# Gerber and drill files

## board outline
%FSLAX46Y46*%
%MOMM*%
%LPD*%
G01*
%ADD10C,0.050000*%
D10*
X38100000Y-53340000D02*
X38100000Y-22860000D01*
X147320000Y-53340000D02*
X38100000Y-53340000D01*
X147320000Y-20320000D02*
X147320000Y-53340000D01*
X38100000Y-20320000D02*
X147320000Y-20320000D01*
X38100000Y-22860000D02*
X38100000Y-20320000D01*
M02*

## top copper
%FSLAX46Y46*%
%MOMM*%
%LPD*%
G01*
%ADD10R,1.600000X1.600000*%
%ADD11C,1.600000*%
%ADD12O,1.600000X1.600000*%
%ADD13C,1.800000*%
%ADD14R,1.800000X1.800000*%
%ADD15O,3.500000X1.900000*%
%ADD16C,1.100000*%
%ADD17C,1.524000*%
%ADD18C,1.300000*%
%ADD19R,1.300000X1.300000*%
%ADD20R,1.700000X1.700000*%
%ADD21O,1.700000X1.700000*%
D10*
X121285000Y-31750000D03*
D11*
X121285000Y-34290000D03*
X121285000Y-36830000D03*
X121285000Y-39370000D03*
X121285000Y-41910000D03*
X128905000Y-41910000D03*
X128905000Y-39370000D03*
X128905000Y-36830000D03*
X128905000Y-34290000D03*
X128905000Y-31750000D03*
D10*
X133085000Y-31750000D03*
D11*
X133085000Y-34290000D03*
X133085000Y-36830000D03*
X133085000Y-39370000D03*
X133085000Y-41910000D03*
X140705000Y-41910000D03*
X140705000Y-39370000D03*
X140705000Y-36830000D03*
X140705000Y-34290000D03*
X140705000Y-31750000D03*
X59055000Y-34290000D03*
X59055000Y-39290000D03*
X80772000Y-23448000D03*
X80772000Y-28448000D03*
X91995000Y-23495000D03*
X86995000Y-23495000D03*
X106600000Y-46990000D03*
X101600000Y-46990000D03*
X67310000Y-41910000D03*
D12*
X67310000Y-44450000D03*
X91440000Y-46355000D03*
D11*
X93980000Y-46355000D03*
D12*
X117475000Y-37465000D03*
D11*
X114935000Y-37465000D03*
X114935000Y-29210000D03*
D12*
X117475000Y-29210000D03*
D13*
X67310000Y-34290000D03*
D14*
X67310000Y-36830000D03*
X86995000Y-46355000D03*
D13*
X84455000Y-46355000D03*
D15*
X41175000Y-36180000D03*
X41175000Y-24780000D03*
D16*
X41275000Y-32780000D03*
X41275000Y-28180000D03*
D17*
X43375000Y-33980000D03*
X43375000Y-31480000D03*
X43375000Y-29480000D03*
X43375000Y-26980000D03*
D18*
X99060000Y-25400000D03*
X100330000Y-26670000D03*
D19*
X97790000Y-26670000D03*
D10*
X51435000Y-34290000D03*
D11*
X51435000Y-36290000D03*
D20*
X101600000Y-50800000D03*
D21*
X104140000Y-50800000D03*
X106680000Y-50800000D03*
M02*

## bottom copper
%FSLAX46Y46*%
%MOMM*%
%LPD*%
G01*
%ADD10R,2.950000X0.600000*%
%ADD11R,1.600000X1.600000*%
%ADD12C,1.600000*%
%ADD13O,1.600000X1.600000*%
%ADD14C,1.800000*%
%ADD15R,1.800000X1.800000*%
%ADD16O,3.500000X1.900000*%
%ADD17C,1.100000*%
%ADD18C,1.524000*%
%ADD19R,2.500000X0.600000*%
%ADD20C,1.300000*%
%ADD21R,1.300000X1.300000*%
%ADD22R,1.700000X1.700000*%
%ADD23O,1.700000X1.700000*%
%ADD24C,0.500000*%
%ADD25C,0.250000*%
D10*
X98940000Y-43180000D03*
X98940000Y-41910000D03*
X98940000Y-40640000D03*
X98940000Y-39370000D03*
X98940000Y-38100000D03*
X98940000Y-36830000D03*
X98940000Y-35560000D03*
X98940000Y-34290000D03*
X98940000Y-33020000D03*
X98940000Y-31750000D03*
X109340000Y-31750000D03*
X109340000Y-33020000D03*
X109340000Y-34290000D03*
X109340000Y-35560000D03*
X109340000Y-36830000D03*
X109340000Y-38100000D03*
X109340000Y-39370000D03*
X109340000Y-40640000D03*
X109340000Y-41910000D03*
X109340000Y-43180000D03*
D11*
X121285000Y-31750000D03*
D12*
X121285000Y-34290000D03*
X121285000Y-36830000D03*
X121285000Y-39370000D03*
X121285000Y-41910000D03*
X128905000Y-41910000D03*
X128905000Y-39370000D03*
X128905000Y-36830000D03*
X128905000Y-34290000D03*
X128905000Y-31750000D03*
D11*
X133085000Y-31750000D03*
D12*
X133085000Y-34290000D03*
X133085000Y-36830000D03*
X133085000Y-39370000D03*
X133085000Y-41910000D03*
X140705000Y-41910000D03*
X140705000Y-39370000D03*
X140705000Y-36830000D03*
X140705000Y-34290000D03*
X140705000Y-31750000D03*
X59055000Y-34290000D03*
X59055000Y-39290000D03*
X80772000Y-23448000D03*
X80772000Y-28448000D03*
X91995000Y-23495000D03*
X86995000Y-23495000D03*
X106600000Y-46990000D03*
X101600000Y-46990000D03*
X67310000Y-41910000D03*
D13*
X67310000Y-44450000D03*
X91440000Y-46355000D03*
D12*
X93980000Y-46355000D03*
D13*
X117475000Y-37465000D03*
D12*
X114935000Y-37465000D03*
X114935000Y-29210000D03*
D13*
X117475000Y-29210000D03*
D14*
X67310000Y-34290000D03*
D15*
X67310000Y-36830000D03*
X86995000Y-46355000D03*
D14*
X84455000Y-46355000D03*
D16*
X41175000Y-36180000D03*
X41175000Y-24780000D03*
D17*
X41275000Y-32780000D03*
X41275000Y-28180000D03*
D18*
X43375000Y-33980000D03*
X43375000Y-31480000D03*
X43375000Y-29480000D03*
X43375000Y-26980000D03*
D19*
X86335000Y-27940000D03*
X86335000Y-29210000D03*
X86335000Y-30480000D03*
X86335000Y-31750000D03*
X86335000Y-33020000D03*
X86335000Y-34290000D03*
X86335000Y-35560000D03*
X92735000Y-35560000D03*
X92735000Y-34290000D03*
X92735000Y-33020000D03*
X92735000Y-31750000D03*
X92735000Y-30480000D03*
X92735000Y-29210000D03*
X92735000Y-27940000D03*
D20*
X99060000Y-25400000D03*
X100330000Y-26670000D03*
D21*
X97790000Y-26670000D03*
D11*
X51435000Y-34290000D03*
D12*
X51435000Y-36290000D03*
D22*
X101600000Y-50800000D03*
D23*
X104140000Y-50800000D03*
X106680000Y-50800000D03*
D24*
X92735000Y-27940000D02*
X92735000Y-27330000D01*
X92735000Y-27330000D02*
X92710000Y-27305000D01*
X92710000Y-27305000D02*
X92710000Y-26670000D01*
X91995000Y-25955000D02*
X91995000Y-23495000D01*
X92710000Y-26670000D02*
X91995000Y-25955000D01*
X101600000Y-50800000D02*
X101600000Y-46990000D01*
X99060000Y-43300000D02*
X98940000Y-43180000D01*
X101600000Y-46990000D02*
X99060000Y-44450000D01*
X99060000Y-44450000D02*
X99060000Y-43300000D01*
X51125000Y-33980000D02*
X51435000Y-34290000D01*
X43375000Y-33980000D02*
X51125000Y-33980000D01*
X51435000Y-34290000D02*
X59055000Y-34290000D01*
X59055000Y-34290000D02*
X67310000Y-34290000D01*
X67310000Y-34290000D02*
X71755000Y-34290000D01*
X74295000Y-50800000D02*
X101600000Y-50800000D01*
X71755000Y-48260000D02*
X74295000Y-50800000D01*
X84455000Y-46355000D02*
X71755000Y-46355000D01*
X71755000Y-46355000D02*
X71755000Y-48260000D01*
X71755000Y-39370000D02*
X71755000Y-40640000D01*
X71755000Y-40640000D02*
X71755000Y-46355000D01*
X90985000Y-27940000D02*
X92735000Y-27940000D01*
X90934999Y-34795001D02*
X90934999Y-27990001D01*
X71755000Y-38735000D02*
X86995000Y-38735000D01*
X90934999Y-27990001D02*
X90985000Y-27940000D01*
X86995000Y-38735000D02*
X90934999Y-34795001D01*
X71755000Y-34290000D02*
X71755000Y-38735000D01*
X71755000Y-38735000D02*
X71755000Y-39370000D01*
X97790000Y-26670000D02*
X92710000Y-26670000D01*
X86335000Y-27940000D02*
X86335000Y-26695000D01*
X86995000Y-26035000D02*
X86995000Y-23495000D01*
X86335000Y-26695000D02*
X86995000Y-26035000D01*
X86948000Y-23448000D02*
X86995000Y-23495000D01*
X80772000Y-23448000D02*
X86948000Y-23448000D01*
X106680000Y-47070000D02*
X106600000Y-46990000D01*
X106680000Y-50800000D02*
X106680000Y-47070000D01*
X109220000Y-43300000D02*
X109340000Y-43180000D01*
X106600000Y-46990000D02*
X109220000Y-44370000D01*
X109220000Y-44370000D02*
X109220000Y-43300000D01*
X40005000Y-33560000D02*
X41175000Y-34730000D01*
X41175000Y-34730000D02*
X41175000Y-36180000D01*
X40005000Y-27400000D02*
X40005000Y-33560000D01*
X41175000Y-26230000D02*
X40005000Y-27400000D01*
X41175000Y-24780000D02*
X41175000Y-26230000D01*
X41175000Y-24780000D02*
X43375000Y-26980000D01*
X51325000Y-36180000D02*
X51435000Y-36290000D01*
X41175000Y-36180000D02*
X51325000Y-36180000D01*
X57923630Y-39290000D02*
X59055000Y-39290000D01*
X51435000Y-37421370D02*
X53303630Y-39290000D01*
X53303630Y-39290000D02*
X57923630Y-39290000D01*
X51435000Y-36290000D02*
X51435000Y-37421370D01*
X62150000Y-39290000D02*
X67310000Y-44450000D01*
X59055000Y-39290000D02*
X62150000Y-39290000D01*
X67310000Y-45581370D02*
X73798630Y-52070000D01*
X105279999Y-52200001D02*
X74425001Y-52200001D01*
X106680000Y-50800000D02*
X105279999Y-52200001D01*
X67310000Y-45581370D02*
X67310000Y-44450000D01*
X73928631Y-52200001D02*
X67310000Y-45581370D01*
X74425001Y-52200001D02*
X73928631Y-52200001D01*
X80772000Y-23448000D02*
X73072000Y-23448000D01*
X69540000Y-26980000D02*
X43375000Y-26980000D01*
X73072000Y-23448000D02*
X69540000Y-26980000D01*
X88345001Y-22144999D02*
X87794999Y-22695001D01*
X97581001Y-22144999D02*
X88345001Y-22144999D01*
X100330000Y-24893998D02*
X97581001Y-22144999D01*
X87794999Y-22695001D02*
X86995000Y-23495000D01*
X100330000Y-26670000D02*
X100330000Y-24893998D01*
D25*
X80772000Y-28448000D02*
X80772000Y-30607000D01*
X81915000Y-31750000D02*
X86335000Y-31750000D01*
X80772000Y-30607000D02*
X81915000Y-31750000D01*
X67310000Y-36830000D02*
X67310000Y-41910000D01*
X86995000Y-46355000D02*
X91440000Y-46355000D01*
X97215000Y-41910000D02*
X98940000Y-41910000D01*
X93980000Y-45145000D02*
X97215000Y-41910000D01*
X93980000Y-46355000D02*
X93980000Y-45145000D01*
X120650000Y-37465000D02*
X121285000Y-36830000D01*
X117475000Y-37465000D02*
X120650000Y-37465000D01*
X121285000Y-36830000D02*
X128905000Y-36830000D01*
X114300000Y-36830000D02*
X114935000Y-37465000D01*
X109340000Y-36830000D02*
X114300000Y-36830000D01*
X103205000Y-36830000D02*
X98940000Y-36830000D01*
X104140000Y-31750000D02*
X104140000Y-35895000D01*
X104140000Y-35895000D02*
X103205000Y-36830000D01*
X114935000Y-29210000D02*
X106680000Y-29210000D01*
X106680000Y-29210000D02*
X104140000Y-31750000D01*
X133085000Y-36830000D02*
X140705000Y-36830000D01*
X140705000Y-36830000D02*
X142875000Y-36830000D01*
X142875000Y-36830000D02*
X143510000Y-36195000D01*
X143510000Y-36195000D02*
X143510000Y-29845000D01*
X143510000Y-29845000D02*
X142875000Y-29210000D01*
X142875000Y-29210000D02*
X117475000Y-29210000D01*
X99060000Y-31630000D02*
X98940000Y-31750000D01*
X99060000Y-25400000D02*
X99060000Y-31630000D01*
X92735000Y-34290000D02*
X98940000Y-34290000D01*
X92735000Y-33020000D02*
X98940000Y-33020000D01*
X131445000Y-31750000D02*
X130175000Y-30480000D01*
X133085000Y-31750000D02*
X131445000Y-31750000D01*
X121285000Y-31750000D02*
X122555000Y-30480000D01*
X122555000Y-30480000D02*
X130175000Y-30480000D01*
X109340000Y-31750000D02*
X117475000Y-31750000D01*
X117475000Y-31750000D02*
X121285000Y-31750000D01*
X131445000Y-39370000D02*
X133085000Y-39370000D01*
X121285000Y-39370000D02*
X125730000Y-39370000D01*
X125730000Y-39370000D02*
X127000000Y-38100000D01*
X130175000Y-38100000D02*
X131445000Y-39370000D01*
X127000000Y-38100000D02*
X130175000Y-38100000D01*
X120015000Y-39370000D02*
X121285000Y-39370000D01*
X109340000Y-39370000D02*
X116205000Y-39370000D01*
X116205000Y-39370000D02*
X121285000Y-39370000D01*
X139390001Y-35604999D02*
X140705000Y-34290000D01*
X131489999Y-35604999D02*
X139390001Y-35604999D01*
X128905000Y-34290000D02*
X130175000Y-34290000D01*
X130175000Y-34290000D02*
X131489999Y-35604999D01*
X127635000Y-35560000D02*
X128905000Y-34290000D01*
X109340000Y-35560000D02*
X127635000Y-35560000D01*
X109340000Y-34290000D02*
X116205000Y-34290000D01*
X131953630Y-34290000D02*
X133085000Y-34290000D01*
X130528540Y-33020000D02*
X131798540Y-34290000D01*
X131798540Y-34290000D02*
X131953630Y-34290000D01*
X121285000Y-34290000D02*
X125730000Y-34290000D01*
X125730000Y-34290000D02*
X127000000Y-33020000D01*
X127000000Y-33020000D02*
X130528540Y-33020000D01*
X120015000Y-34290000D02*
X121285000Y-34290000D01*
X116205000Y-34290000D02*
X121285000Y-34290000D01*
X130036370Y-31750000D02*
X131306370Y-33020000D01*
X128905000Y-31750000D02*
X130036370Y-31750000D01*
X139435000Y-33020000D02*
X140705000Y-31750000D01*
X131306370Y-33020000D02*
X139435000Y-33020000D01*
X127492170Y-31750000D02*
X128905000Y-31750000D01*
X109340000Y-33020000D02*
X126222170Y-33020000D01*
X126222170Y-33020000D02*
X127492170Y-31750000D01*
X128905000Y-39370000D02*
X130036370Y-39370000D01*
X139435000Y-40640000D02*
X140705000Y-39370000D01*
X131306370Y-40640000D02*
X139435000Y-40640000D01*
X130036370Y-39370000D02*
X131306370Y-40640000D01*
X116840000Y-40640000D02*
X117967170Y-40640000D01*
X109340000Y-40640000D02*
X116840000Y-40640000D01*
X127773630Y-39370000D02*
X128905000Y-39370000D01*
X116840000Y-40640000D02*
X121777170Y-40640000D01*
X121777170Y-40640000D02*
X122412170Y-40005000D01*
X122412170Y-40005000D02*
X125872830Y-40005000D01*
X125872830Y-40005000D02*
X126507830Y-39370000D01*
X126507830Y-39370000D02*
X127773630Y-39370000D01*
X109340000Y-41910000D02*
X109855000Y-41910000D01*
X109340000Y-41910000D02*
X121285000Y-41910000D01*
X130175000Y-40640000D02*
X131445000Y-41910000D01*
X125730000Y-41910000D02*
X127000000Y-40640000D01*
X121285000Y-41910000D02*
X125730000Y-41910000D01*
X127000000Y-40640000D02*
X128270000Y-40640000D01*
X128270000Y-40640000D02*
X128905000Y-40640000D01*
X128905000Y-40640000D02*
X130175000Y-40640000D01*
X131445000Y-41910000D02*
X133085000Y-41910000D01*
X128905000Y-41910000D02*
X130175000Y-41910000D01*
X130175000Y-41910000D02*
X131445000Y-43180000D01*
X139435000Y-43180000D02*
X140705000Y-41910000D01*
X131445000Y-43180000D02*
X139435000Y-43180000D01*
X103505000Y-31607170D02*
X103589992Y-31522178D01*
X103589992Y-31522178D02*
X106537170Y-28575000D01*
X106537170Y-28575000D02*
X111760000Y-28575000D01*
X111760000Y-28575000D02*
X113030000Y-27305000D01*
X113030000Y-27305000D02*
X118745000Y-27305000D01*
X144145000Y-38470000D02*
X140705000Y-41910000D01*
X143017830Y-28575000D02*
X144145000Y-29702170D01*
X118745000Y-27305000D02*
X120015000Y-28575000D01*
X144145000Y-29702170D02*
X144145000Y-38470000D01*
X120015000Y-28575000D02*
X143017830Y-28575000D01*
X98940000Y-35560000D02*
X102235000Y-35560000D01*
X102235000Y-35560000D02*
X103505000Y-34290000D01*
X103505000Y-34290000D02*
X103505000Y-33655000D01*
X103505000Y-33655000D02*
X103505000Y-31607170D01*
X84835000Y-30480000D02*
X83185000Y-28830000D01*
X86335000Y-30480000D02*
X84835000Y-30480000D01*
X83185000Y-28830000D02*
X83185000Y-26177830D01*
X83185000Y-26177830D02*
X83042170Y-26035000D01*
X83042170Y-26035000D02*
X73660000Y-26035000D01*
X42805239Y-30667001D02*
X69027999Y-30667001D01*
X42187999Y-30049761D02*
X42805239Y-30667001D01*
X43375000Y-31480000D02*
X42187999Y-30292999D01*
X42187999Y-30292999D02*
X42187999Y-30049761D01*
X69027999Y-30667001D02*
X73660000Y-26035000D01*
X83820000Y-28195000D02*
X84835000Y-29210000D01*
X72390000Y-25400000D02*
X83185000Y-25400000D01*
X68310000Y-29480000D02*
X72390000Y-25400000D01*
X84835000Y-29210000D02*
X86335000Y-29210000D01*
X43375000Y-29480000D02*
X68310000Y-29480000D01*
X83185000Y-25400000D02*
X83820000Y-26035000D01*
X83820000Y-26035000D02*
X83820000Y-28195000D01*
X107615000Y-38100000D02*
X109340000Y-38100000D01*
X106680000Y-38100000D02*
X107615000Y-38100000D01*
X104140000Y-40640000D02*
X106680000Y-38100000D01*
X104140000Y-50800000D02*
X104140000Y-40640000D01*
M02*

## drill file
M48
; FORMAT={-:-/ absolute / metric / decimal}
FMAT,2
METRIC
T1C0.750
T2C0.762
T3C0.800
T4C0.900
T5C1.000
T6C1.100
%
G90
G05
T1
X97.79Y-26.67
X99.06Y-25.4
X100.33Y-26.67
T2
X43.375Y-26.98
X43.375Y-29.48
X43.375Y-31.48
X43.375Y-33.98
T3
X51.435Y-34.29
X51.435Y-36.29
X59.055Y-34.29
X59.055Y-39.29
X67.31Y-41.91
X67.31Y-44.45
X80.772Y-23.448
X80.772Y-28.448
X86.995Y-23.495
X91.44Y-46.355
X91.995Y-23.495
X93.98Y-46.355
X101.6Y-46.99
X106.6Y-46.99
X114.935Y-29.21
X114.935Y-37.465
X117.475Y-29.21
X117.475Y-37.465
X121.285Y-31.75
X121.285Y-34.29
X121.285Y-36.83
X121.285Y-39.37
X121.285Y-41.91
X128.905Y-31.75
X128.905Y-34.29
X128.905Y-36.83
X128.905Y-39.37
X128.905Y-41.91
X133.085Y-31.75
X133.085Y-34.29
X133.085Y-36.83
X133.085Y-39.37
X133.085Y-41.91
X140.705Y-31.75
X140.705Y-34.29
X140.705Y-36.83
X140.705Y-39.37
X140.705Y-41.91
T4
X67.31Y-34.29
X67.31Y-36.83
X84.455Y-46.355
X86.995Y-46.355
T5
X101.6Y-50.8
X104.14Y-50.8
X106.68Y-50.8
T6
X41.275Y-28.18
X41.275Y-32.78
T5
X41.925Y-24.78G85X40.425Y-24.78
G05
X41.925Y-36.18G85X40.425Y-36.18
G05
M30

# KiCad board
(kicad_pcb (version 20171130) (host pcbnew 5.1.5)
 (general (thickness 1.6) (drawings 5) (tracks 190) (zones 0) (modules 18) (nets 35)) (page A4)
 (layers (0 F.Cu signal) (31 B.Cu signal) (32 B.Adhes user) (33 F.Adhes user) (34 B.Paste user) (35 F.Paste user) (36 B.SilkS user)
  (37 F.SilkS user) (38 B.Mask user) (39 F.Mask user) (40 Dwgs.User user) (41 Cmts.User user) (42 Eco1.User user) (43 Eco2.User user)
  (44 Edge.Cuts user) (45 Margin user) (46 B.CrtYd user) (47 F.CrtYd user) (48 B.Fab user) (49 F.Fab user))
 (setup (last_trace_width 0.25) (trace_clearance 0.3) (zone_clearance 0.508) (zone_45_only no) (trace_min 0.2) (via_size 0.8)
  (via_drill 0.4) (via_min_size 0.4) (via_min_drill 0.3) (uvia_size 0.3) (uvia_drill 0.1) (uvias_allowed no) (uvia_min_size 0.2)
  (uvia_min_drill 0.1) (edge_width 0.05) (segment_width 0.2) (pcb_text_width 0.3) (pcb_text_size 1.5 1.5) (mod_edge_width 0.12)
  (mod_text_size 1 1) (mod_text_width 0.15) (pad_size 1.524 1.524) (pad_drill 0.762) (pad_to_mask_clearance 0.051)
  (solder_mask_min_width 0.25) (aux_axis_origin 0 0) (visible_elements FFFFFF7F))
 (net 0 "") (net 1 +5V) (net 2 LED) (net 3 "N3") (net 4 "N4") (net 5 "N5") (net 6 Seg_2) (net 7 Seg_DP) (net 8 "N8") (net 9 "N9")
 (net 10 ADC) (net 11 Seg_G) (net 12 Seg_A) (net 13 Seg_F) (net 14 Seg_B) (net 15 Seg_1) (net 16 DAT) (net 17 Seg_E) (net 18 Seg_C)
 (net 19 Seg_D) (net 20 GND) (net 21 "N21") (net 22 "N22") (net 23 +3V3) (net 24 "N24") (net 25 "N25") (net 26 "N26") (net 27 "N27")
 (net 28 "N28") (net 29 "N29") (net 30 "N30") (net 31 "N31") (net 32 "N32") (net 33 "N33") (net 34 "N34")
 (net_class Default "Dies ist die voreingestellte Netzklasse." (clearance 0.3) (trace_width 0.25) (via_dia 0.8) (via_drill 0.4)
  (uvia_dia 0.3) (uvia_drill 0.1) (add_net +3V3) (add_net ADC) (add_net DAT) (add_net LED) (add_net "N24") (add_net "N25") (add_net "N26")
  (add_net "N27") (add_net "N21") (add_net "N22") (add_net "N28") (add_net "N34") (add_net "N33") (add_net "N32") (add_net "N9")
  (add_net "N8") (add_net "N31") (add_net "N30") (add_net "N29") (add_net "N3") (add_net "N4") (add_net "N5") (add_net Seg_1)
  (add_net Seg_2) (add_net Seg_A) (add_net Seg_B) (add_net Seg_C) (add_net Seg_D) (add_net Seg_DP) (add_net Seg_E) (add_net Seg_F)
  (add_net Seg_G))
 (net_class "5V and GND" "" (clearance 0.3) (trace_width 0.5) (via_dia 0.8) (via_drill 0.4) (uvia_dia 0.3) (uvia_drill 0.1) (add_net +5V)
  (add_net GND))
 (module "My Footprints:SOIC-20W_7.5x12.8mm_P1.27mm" (layer B.Cu) (at 104.14 37.465)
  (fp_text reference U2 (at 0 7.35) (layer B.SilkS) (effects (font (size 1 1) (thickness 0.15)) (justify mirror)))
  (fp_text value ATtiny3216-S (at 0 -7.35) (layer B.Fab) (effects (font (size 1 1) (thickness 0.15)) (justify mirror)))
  (pad 1 smd rect (at -5.2 5.715) (size 2.95 0.6) (layers B.Cu B.Paste B.Mask) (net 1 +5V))
  (pad 2 smd rect (at -5.2 4.445) (size 2.95 0.6) (layers B.Cu B.Paste B.Mask) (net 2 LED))
  (pad 3 smd rect (at -5.2 3.175) (size 2.95 0.6) (layers B.Cu B.Paste B.Mask) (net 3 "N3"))
  (pad 4 smd rect (at -5.2 1.905) (size 2.95 0.6) (layers B.Cu B.Paste B.Mask) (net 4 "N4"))
  (pad 5 smd rect (at -5.2 0.635) (size 2.95 0.6) (layers B.Cu B.Paste B.Mask) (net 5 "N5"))
  (pad 6 smd rect (at -5.2 -0.635) (size 2.95 0.6) (layers B.Cu B.Paste B.Mask) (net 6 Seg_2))
  (pad 7 smd rect (at -5.2 -1.905) (size 2.95 0.6) (layers B.Cu B.Paste B.Mask) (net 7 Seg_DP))
  (pad 8 smd rect (at -5.2 -3.175) (size 2.95 0.6) (layers B.Cu B.Paste B.Mask) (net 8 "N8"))
  (pad 9 smd rect (at -5.2 -4.445) (size 2.95 0.6) (layers B.Cu B.Paste B.Mask) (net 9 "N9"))
  (pad 10 smd rect (at -5.2 -5.715) (size 2.95 0.6) (layers B.Cu B.Paste B.Mask) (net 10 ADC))
  (pad 11 smd rect (at 5.2 -5.715) (size 2.95 0.6) (layers B.Cu B.Paste B.Mask) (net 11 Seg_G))
  (pad 12 smd rect (at 5.2 -4.445) (size 2.95 0.6) (layers B.Cu B.Paste B.Mask) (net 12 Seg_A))
  (pad 13 smd rect (at 5.2 -3.175) (size 2.95 0.6) (layers B.Cu B.Paste B.Mask) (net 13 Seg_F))
  (pad 14 smd rect (at 5.2 -1.905) (size 2.95 0.6) (layers B.Cu B.Paste B.Mask) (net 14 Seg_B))
  (pad 15 smd rect (at 5.2 -0.635) (size 2.95 0.6) (layers B.Cu B.Paste B.Mask) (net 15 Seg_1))
  (pad 16 smd rect (at 5.2 0.635) (size 2.95 0.6) (layers B.Cu B.Paste B.Mask) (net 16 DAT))
  (pad 17 smd rect (at 5.2 1.905) (size 2.95 0.6) (layers B.Cu B.Paste B.Mask) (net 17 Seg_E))
  (pad 18 smd rect (at 5.2 3.175) (size 2.95 0.6) (layers B.Cu B.Paste B.Mask) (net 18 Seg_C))
  (pad 19 smd rect (at 5.2 4.445) (size 2.95 0.6) (layers B.Cu B.Paste B.Mask) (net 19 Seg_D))
  (pad 20 smd rect (at 5.2 5.715) (size 2.95 0.6) (layers B.Cu B.Paste B.Mask) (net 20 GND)))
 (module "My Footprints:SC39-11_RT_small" (layer F.Cu) (at 121.285 31.75)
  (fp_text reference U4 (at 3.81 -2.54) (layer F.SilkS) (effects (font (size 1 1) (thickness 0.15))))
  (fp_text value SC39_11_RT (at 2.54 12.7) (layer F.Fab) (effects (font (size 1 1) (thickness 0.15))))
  (pad 1 thru_hole rect (at 0 0) (size 1.6 1.6) (drill 0.8) (layers *.Cu *.Mask) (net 11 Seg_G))
  (pad 2 thru_hole circle (at 0 2.54) (size 1.6 1.6) (drill 0.8) (layers *.Cu *.Mask) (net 13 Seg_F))
  (pad 3 thru_hole circle (at 0 5.08) (size 1.6 1.6) (drill 0.8) (layers *.Cu *.Mask) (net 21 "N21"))
  (pad 4 thru_hole circle (at 0 7.62) (size 1.6 1.6) (drill 0.8) (layers *.Cu *.Mask) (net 17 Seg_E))
  (pad 5 thru_hole circle (at 0 10.16) (size 1.6 1.6) (drill 0.8) (layers *.Cu *.Mask) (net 19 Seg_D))
  (pad 6 thru_hole circle (at 7.62 10.16) (size 1.6 1.6) (drill 0.8) (layers *.Cu *.Mask) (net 7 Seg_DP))
  (pad 7 thru_hole circle (at 7.62 7.62) (size 1.6 1.6) (drill 0.8) (layers *.Cu *.Mask) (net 18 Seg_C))
  (pad 8 thru_hole circle (at 7.62 5.08) (size 1.6 1.6) (drill 0.8) (layers *.Cu *.Mask) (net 21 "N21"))
  (pad 9 thru_hole circle (at 7.62 2.54) (size 1.6 1.6) (drill 0.8) (layers *.Cu *.Mask) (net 14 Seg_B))
  (pad 10 thru_hole circle (at 7.62 0) (size 1.6 1.6) (drill 0.8) (layers *.Cu *.Mask) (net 12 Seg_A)))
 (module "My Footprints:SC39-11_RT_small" (layer F.Cu) (at 133.085 31.75)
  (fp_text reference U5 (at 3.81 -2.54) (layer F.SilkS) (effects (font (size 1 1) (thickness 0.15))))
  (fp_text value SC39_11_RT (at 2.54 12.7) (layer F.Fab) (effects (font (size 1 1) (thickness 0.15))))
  (pad 1 thru_hole rect (at 0 0) (size 1.6 1.6) (drill 0.8) (layers *.Cu *.Mask) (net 11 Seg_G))
  (pad 2 thru_hole circle (at 0 2.54) (size 1.6 1.6) (drill 0.8) (layers *.Cu *.Mask) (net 13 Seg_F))
  (pad 3 thru_hole circle (at 0 5.08) (size 1.6 1.6) (drill 0.8) (layers *.Cu *.Mask) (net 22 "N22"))
  (pad 4 thru_hole circle (at 0 7.62) (size 1.6 1.6) (drill 0.8) (layers *.Cu *.Mask) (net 17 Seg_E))
  (pad 5 thru_hole circle (at 0 10.16) (size 1.6 1.6) (drill 0.8) (layers *.Cu *.Mask) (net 19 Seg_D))
  (pad 6 thru_hole circle (at 7.62 10.16) (size 1.6 1.6) (drill 0.8) (layers *.Cu *.Mask) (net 7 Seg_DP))
  (pad 7 thru_hole circle (at 7.62 7.62) (size 1.6 1.6) (drill 0.8) (layers *.Cu *.Mask) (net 18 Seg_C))
  (pad 8 thru_hole circle (at 7.62 5.08) (size 1.6 1.6) (drill 0.8) (layers *.Cu *.Mask) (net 22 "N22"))
  (pad 9 thru_hole circle (at 7.62 2.54) (size 1.6 1.6) (drill 0.8) (layers *.Cu *.Mask) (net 14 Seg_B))
  (pad 10 thru_hole circle (at 7.62 0) (size 1.6 1.6) (drill 0.8) (layers *.Cu *.Mask) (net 12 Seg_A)))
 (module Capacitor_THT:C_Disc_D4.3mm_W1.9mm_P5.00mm (layer F.Cu) (at 59.055 34.29 270)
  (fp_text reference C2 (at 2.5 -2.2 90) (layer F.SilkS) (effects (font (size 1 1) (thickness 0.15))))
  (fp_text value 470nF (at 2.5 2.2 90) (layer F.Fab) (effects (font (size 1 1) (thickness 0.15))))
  (pad 1 thru_hole circle (at 0 0 270) (size 1.6 1.6) (drill 0.8) (layers *.Cu *.Mask) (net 1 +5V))
  (pad 2 thru_hole circle (at 5 0 270) (size 1.6 1.6) (drill 0.8) (layers *.Cu *.Mask) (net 20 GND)))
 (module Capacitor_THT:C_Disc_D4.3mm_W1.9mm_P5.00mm (layer F.Cu) (at 80.772 28.448 90)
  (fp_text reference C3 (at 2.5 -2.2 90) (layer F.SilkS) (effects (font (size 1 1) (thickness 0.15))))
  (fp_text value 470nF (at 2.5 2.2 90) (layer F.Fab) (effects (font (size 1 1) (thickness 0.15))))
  (pad 2 thru_hole circle (at 5 0 90) (size 1.6 1.6) (drill 0.8) (layers *.Cu *.Mask) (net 20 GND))
  (pad 1 thru_hole circle (at 0 0 90) (size 1.6 1.6) (drill 0.8) (layers *.Cu *.Mask) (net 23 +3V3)))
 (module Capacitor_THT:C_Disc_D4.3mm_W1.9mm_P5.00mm (layer F.Cu) (at 86.995 23.495)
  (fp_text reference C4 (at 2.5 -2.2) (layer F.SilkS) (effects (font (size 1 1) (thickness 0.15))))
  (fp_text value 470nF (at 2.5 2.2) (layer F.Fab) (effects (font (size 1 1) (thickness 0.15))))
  (pad 2 thru_hole circle (at 5 0) (size 1.6 1.6) (drill 0.8) (layers *.Cu *.Mask) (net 1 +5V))
  (pad 1 thru_hole circle (at 0 0) (size 1.6 1.6) (drill 0.8) (layers *.Cu *.Mask) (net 20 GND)))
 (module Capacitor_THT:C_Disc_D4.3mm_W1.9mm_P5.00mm (layer F.Cu) (at 106.6 46.99 180)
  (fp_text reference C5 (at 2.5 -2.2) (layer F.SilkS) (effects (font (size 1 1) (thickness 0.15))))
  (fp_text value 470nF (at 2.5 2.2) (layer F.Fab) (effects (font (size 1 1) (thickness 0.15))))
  (pad 1 thru_hole circle (at 0 0 180) (size 1.6 1.6) (drill 0.8) (layers *.Cu *.Mask) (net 20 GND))
  (pad 2 thru_hole circle (at 5 0 180) (size 1.6 1.6) (drill 0.8) (layers *.Cu *.Mask) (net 1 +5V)))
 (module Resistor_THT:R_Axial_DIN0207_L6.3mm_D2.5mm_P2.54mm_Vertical (layer F.Cu) (at 67.31 41.91 270)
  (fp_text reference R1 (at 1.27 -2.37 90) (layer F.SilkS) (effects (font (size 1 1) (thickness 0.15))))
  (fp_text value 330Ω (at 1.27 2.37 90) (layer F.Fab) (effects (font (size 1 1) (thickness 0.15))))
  (pad 1 thru_hole circle (at 0 0 270) (size 1.6 1.6) (drill 0.8) (layers *.Cu *.Mask) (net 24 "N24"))
  (pad 2 thru_hole oval (at 2.54 0 270) (size 1.6 1.6) (drill 0.8) (layers *.Cu *.Mask) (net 20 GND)))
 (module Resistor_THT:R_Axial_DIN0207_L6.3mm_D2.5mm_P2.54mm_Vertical (layer F.Cu) (at 93.98 46.355 180)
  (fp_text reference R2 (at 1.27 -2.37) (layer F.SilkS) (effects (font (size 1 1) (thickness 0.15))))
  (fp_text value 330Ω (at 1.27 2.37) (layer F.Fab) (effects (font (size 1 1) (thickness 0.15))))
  (pad 2 thru_hole oval (at 2.54 0 180) (size 1.6 1.6) (drill 0.8) (layers *.Cu *.Mask) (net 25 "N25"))
  (pad 1 thru_hole circle (at 0 0 180) (size 1.6 1.6) (drill 0.8) (layers *.Cu *.Mask) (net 2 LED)))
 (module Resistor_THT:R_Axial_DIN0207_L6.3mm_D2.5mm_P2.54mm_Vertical (layer F.Cu) (at 114.935 37.465)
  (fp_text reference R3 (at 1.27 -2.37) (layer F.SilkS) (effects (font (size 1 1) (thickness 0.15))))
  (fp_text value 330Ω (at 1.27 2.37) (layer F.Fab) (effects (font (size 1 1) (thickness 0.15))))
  (pad 2 thru_hole oval (at 2.54 0) (size 1.6 1.6) (drill 0.8) (layers *.Cu *.Mask) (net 21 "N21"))
  (pad 1 thru_hole circle (at 0 0) (size 1.6 1.6) (drill 0.8) (layers *.Cu *.Mask) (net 15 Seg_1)))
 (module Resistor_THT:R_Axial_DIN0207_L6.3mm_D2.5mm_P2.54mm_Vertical (layer F.Cu) (at 114.935 29.21)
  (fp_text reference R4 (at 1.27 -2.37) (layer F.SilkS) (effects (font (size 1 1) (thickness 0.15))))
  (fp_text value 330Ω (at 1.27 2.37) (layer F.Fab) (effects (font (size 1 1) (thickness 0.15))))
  (pad 1 thru_hole circle (at 0 0) (size 1.6 1.6) (drill 0.8) (layers *.Cu *.Mask) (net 6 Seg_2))
  (pad 2 thru_hole oval (at 2.54 0) (size 1.6 1.6) (drill 0.8) (layers *.Cu *.Mask) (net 22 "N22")))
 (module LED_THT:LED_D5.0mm (layer F.Cu) (at 67.31 36.83 90)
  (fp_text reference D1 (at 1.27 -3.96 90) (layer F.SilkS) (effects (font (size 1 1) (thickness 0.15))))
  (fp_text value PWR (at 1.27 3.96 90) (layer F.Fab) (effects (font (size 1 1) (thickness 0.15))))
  (pad 2 thru_hole circle (at 2.54 0 90) (size 1.8 1.8) (drill 0.9) (layers *.Cu *.Mask) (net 1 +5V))
  (pad 1 thru_hole rect (at 0 0 90) (size 1.8 1.8) (drill 0.9) (layers *.Cu *.Mask) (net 24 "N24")))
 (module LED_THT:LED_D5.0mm (layer F.Cu) (at 86.995 46.355 180)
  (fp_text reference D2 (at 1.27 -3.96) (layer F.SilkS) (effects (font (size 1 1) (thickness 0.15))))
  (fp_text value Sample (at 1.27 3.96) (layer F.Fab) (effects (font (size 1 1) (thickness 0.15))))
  (pad 1 thru_hole rect (at 0 0 180) (size 1.8 1.8) (drill 0.9) (layers *.Cu *.Mask) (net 25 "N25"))
  (pad 2 thru_hole circle (at 2.54 0 180) (size 1.8 1.8) (drill 0.9) (layers *.Cu *.Mask) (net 1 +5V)))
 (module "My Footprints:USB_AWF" (layer F.Cu) (at 41.275 30.48 180)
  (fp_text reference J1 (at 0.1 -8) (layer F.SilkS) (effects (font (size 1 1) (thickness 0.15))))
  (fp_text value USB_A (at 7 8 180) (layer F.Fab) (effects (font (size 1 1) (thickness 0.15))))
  (pad 5 thru_hole oval (at 0.1 -5.7 180) (size 3.5 1.9) (drill oval 2.5 1) (layers *.Cu *.Mask) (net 20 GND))
  (pad 5 thru_hole oval (at 0.1 5.7 180) (size 3.5 1.9) (drill oval 2.5 1) (layers *.Cu *.Mask) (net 20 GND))
  (pad "" thru_hole circle (at 0 -2.3 180) (size 1.1 1.1) (drill 1.1) (layers *.Cu *.Mask))
  (pad "" thru_hole circle (at 0 2.3 180) (size 1.1 1.1) (drill 1.1) (layers *.Cu *.Mask))
  (pad 1 thru_hole circle (at -2.1 -3.5 180) (size 1.524 1.524) (drill 0.762) (layers *.Cu *.Mask) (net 1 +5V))
  (pad 2 thru_hole circle (at -2.1 -1 180) (size 1.524 1.524) (drill 0.762) (layers *.Cu *.Mask) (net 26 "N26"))
  (pad 3 thru_hole circle (at -2.1 1 180) (size 1.524 1.524) (drill 0.762) (layers *.Cu *.Mask) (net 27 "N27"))
  (pad 4 thru_hole circle (at -2.1 3.5 180) (size 1.524 1.524) (drill 0.762) (layers *.Cu *.Mask) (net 20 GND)))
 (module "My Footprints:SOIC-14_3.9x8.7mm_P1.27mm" (layer B.Cu) (at 89.535 31.75 180)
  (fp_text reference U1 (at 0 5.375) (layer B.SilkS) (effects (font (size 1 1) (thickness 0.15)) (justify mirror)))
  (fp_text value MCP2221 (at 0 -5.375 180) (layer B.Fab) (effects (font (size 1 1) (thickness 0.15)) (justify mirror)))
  (pad 14 smd rect (at 3.2 3.81 180) (size 2.5 0.6) (layers B.Cu B.Paste B.Mask) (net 20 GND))
  (pad 13 smd rect (at 3.2 2.54 180) (size 2.5 0.6) (layers B.Cu B.Paste B.Mask) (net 27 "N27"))
  (pad 12 smd rect (at 3.2 1.27 180) (size 2.5 0.6) (layers B.Cu B.Paste B.Mask) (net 26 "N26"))
  (pad 11 smd rect (at 3.2 0 180) (size 2.5 0.6) (layers B.Cu B.Paste B.Mask) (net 23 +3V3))
  (pad 10 smd rect (at 3.2 -1.27 180) (size 2.5 0.6) (layers B.Cu B.Paste B.Mask) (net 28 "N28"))
  (pad 9 smd rect (at 3.2 -2.54 180) (size 2.5 0.6) (layers B.Cu B.Paste B.Mask) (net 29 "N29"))
  (pad 8 smd rect (at 3.2 -3.81 180) (size 2.5 0.6) (layers B.Cu B.Paste B.Mask) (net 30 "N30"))
  (pad 7 smd rect (at -3.2 -3.81 180) (size 2.5 0.6) (layers B.Cu B.Paste B.Mask) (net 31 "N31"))
  (pad 6 smd rect (at -3.2 -2.54 180) (size 2.5 0.6) (layers B.Cu B.Paste B.Mask) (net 8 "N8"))
  (pad 5 smd rect (at -3.2 -1.27 180) (size 2.5 0.6) (layers B.Cu B.Paste B.Mask) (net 9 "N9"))
  (pad 4 smd rect (at -3.2 0 180) (size 2.5 0.6) (layers B.Cu B.Paste B.Mask) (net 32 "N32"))
  (pad 3 smd rect (at -3.2 1.27 180) (size 2.5 0.6) (layers B.Cu B.Paste B.Mask) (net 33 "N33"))
  (pad 2 smd rect (at -3.2 2.54 180) (size 2.5 0.6) (layers B.Cu B.Paste B.Mask) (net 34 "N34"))
  (pad 1 smd rect (at -3.2 3.81 180) (size 2.5 0.6) (layers B.Cu B.Paste B.Mask) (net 1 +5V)))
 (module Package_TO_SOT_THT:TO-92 (layer F.Cu) (at 97.79 26.67)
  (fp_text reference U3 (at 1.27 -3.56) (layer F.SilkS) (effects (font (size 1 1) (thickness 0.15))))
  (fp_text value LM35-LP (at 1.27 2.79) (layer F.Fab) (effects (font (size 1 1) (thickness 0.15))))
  (pad 2 thru_hole circle (at 1.27 -1.27 90) (size 1.3 1.3) (drill 0.75) (layers *.Cu *.Mask) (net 10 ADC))
  (pad 3 thru_hole circle (at 2.54 0 90) (size 1.3 1.3) (drill 0.75) (layers *.Cu *.Mask) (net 20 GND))
  (pad 1 thru_hole rect (at 0 0 90) (size 1.3 1.3) (drill 0.75) (layers *.Cu *.Mask) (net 1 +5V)))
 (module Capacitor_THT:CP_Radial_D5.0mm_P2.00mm (layer F.Cu) (at 51.435 34.29 270)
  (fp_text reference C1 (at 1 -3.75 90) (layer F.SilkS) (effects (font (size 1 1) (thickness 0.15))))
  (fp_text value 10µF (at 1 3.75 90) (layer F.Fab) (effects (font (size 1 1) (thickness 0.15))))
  (pad 1 thru_hole rect (at 0 0 270) (size 1.6 1.6) (drill 0.8) (layers *.Cu *.Mask) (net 1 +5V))
  (pad 2 thru_hole circle (at 2 0 270) (size 1.6 1.6) (drill 0.8) (layers *.Cu *.Mask) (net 20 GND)))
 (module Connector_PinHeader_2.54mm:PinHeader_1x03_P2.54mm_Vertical (layer F.Cu) (at 101.6 50.8 90)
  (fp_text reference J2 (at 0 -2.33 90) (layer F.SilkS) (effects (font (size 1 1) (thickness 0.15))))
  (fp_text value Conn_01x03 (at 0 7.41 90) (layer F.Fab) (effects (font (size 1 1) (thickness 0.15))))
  (pad 1 thru_hole rect (at 0 0 90) (size 1.7 1.7) (drill 1) (layers *.Cu *.Mask) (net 1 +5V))
  (pad 2 thru_hole oval (at 0 2.54 90) (size 1.7 1.7) (drill 1) (layers *.Cu *.Mask) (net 16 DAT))
  (pad 3 thru_hole oval (at 0 5.08 90) (size 1.7 1.7) (drill 1) (layers *.Cu *.Mask) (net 20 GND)))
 (gr_line (start 38.1 53.34) (end 38.1 22.86) (layer Edge.Cuts) (width 0.05))
 (gr_line (start 147.32 53.34) (end 38.1 53.34) (layer Edge.Cuts) (width 0.05))
 (gr_line (start 147.32 20.32) (end 147.32 53.34) (layer Edge.Cuts) (width 0.05))
 (gr_line (start 38.1 20.32) (end 147.32 20.32) (layer Edge.Cuts) (width 0.05))
 (gr_line (start 38.1 22.86) (end 38.1 20.32) (layer Edge.Cuts) (width 0.05))
 (segment (start 92.735 27.94) (end 92.735 27.33) (width 0.5) (layer B.Cu) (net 1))
 (segment (start 92.735 27.33) (end 92.71 27.305) (width 0.5) (layer B.Cu) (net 1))
 (segment (start 92.71 27.305) (end 92.71 26.67) (width 0.5) (layer B.Cu) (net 1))
 (segment (start 91.995 25.955) (end 91.995 23.495) (width 0.5) (layer B.Cu) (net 1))
 (segment (start 92.71 26.67) (end 91.995 25.955) (width 0.5) (layer B.Cu) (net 1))
 (segment (start 101.6 50.8) (end 101.6 46.99) (width 0.5) (layer B.Cu) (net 1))
 (segment (start 99.06 43.3) (end 98.94 43.18) (width 0.5) (layer B.Cu) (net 1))
 (segment (start 101.6 46.99) (end 99.06 44.45) (width 0.5) (layer B.Cu) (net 1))
 (segment (start 99.06 44.45) (end 99.06 43.3) (width 0.5) (layer B.Cu) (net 1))
 (segment (start 51.125 33.98) (end 51.435 34.29) (width 0.5) (layer B.Cu) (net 1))
 (segment (start 43.375 33.98) (end 51.125 33.98) (width 0.5) (layer B.Cu) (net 1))
 (segment (start 51.435 34.29) (end 59.055 34.29) (width 0.5) (layer B.Cu) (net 1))
 (segment (start 59.055 34.29) (end 67.31 34.29) (width 0.5) (layer B.Cu) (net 1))
 (segment (start 67.31 34.29) (end 71.755 34.29) (width 0.5) (layer B.Cu) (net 1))
 (segment (start 74.295 50.8) (end 101.6 50.8) (width 0.5) (layer B.Cu) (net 1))
 (segment (start 71.755 48.26) (end 74.295 50.8) (width 0.5) (layer B.Cu) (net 1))
 (segment (start 84.455 46.355) (end 71.755 46.355) (width 0.5) (layer B.Cu) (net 1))
 (segment (start 71.755 46.355) (end 71.755 48.26) (width 0.5) (layer B.Cu) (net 1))
 (segment (start 71.755 39.37) (end 71.755 40.64) (width 0.5) (layer B.Cu) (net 1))
 (segment (start 71.755 40.64) (end 71.755 46.355) (width 0.5) (layer B.Cu) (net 1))
 (segment (start 90.985 27.94) (end 92.735 27.94) (width 0.5) (layer B.Cu) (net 1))
 (segment (start 90.934999 34.795001) (end 90.934999 27.990001) (width 0.5) (layer B.Cu) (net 1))
 (segment (start 71.755 38.735) (end 86.995 38.735) (width 0.5) (layer B.Cu) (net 1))
 (segment (start 90.934999 27.990001) (end 90.985 27.94) (width 0.5) (layer B.Cu) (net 1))
 (segment (start 86.995 38.735) (end 90.934999 34.795001) (width 0.5) (layer B.Cu) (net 1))
 (segment (start 71.755 34.29) (end 71.755 38.735) (width 0.5) (layer B.Cu) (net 1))
 (segment (start 71.755 38.735) (end 71.755 39.37) (width 0.5) (layer B.Cu) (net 1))
 (segment (start 97.79 26.67) (end 92.71 26.67) (width 0.5) (layer B.Cu) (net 1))
 (segment (start 86.335 27.94) (end 86.335 26.695) (width 0.5) (layer B.Cu) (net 20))
 (segment (start 86.995 26.035) (end 86.995 23.495) (width 0.5) (layer B.Cu) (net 20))
 (segment (start 86.335 26.695) (end 86.995 26.035) (width 0.5) (layer B.Cu) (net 20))
 (segment (start 86.948 23.448) (end 86.995 23.495) (width 0.5) (layer B.Cu) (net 20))
 (segment (start 80.772 23.448) (end 86.948 23.448) (width 0.5) (layer B.Cu) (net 20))
 (segment (start 106.68 47.07) (end 106.6 46.99) (width 0.5) (layer B.Cu) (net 20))
 (segment (start 106.68 50.8) (end 106.68 47.07) (width 0.5) (layer B.Cu) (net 20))
 (segment (start 109.22 43.3) (end 109.34 43.18) (width 0.5) (layer B.Cu) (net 20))
 (segment (start 106.6 46.99) (end 109.22 44.37) (width 0.5) (layer B.Cu) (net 20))
 (segment (start 109.22 44.37) (end 109.22 43.3) (width 0.5) (layer B.Cu) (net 20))
 (segment (start 40.005 33.56) (end 41.175 34.73) (width 0.5) (layer B.Cu) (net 20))
 (segment (start 41.175 34.73) (end 41.175 36.18) (width 0.5) (layer B.Cu) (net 20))
 (segment (start 40.005 27.4) (end 40.005 33.56) (width 0.5) (layer B.Cu) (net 20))
 (segment (start 41.175 26.23) (end 40.005 27.4) (width 0.5) (layer B.Cu) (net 20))
 (segment (start 41.175 24.78) (end 41.175 26.23) (width 0.5) (layer B.Cu) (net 20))
 (segment (start 41.175 24.78) (end 43.375 26.98) (width 0.5) (layer B.Cu) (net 20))
 (segment (start 51.325 36.18) (end 51.435 36.29) (width 0.5) (layer B.Cu) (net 20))
 (segment (start 41.175 36.18) (end 51.325 36.18) (width 0.5) (layer B.Cu) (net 20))
 (segment (start 57.92363 39.29) (end 59.055 39.29) (width 0.5) (layer B.Cu) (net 20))
 (segment (start 51.435 37.42137) (end 53.30363 39.29) (width 0.5) (layer B.Cu) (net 20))
 (segment (start 53.30363 39.29) (end 57.92363 39.29) (width 0.5) (layer B.Cu) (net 20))
 (segment (start 51.435 36.29) (end 51.435 37.42137) (width 0.5) (layer B.Cu) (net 20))
 (segment (start 62.15 39.29) (end 67.31 44.45) (width 0.5) (layer B.Cu) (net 20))
 (segment (start 59.055 39.29) (end 62.15 39.29) (width 0.5) (layer B.Cu) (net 20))
 (segment (start 67.31 45.58137) (end 73.79863 52.07) (width 0.5) (layer B.Cu) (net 20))
 (segment (start 105.279999 52.200001) (end 74.425001 52.200001) (width 0.5) (layer B.Cu) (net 20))
 (segment (start 106.68 50.8) (end 105.279999 52.200001) (width 0.5) (layer B.Cu) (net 20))
 (segment (start 67.31 45.58137) (end 67.31 44.45) (width 0.5) (layer B.Cu) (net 20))
 (segment (start 73.928631 52.200001) (end 67.31 45.58137) (width 0.5) (layer B.Cu) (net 20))
 (segment (start 74.425001 52.200001) (end 73.928631 52.200001) (width 0.5) (layer B.Cu) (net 20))
 (segment (start 80.772 23.448) (end 73.072 23.448) (width 0.5) (layer B.Cu) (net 20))
 (segment (start 69.54 26.98) (end 43.375 26.98) (width 0.5) (layer B.Cu) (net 20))
 (segment (start 73.072 23.448) (end 69.54 26.98) (width 0.5) (layer B.Cu) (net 20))
 (segment (start 88.345001 22.144999) (end 87.794999 22.695001) (width 0.5) (layer B.Cu) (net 20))
 (segment (start 97.581001 22.144999) (end 88.345001 22.144999) (width 0.5) (layer B.Cu) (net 20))
 (segment (start 100.33 24.893998) (end 97.581001 22.144999) (width 0.5) (layer B.Cu) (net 20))
 (segment (start 87.794999 22.695001) (end 86.995 23.495) (width 0.5) (layer B.Cu) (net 20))
 (segment (start 100.33 26.67) (end 100.33 24.893998) (width 0.5) (layer B.Cu) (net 20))
 (segment (start 80.772 28.448) (end 80.772 30.607) (width 0.25) (layer B.Cu) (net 23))
 (segment (start 81.915 31.75) (end 86.335 31.75) (width 0.25) (layer B.Cu) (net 23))
 (segment (start 80.772 30.607) (end 81.915 31.75) (width 0.25) (layer B.Cu) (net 23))
 (segment (start 67.31 36.83) (end 67.31 41.91) (width 0.25) (layer B.Cu) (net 24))
 (segment (start 86.995 46.355) (end 91.44 46.355) (width 0.25) (layer B.Cu) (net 25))
 (segment (start 97.215 41.91) (end 98.94 41.91) (width 0.25) (layer B.Cu) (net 2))
 (segment (start 93.98 45.145) (end 97.215 41.91) (width 0.25) (layer B.Cu) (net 2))
 (segment (start 93.98 46.355) (end 93.98 45.145) (width 0.25) (layer B.Cu) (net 2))
 (segment (start 120.65 37.465) (end 121.285 36.83) (width 0.25) (layer B.Cu) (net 21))
 (segment (start 117.475 37.465) (end 120.65 37.465) (width 0.25) (layer B.Cu) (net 21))
 (segment (start 121.285 36.83) (end 128.905 36.83) (width 0.25) (layer B.Cu) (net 21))
 (segment (start 114.3 36.83) (end 114.935 37.465) (width 0.25) (layer B.Cu) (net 15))
 (segment (start 109.34 36.83) (end 114.3 36.83) (width 0.25) (layer B.Cu) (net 15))
 (segment (start 103.205 36.83) (end 98.94 36.83) (width 0.25) (layer B.Cu) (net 6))
 (segment (start 104.14 31.75) (end 104.14 35.895) (width 0.25) (layer B.Cu) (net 6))
 (segment (start 104.14 35.895) (end 103.205 36.83) (width 0.25) (layer B.Cu) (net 6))
 (segment (start 114.935 29.21) (end 106.68 29.21) (width 0.25) (layer B.Cu) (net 6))
 (segment (start 106.68 29.21) (end 104.14 31.75) (width 0.25) (layer B.Cu) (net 6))
 (segment (start 133.085 36.83) (end 140.705 36.83) (width 0.25) (layer B.Cu) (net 22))
 (segment (start 140.705 36.83) (end 142.875 36.83) (width 0.25) (layer B.Cu) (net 22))
 (segment (start 142.875 36.83) (end 143.51 36.195) (width 0.25) (layer B.Cu) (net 22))
 (segment (start 143.51 36.195) (end 143.51 29.845) (width 0.25) (layer B.Cu) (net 22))
 (segment (start 143.51 29.845) (end 142.875 29.21) (width 0.25) (layer B.Cu) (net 22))
 (segment (start 142.875 29.21) (end 117.475 29.21) (width 0.25) (layer B.Cu) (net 22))
 (segment (start 99.06 31.63) (end 98.94 31.75) (width 0.25) (layer B.Cu) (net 10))
 (segment (start 99.06 25.4) (end 99.06 31.63) (width 0.25) (layer B.Cu) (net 10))
 (segment (start 92.735 34.29) (end 98.94 34.29) (width 0.25) (layer B.Cu) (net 8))
 (segment (start 92.735 33.02) (end 98.94 33.02) (width 0.25) (layer B.Cu) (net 9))
 (segment (start 131.445 31.75) (end 130.175 30.48) (width 0.25) (layer B.Cu) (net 11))
 (segment (start 133.085 31.75) (end 131.445 31.75) (width 0.25) (layer B.Cu) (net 11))
 (segment (start 121.285 31.75) (end 122.555 30.48) (width 0.25) (layer B.Cu) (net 11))
 (segment (start 122.555 30.48) (end 130.175 30.48) (width 0.25) (layer B.Cu) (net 11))
 (segment (start 109.34 31.75) (end 117.475 31.75) (width 0.25) (layer B.Cu) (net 11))
 (segment (start 117.475 31.75) (end 121.285 31.75) (width 0.25) (layer B.Cu) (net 11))
 (segment (start 131.445 39.37) (end 133.085 39.37) (width 0.25) (layer B.Cu) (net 17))
 (segment (start 121.285 39.37) (end 125.73 39.37) (width 0.25) (layer B.Cu) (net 17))
 (segment (start 125.73 39.37) (end 127 38.1) (width 0.25) (layer B.Cu) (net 17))
 (segment (start 130.175 38.1) (end 131.445 39.37) (width 0.25) (layer B.Cu) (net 17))
 (segment (start 127 38.1) (end 130.175 38.1) (width 0.25) (layer B.Cu) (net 17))
 (segment (start 120.015 39.37) (end 121.285 39.37) (width 0.25) (layer B.Cu) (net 17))
 (segment (start 109.34 39.37) (end 116.205 39.37) (width 0.25) (layer B.Cu) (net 17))
 (segment (start 116.205 39.37) (end 121.285 39.37) (width 0.25) (layer B.Cu) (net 17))
 (segment (start 139.390001 35.604999) (end 140.705 34.29) (width 0.25) (layer B.Cu) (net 14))
 (segment (start 131.489999 35.604999) (end 139.390001 35.604999) (width 0.25) (layer B.Cu) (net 14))
 (segment (start 128.905 34.29) (end 130.175 34.29) (width 0.25) (layer B.Cu) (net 14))
 (segment (start 130.175 34.29) (end 131.489999 35.604999) (width 0.25) (layer B.Cu) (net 14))
 (segment (start 127.635 35.56) (end 128.905 34.29) (width 0.25) (layer B.Cu) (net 14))
 (segment (start 109.34 35.56) (end 127.635 35.56) (width 0.25) (layer B.Cu) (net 14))
 (segment (start 109.34 34.29) (end 116.205 34.29) (width 0.25) (layer B.Cu) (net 13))
 (segment (start 131.95363 34.29) (end 133.085 34.29) (width 0.25) (layer B.Cu) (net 13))
 (segment (start 130.52854 33.02) (end 131.79854 34.29) (width 0.25) (layer B.Cu) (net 13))
 (segment (start 131.79854 34.29) (end 131.95363 34.29) (width 0.25) (layer B.Cu) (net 13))
 (segment (start 121.285 34.29) (end 125.73 34.29) (width 0.25) (layer B.Cu) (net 13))
 (segment (start 125.73 34.29) (end 127 33.02) (width 0.25) (layer B.Cu) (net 13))
 (segment (start 127 33.02) (end 130.52854 33.02) (width 0.25) (layer B.Cu) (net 13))
 (segment (start 120.015 34.29) (end 121.285 34.29) (width 0.25) (layer B.Cu) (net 13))
 (segment (start 116.205 34.29) (end 121.285 34.29) (width 0.25) (layer B.Cu) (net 13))
 (segment (start 130.03637 31.75) (end 131.30637 33.02) (width 0.25) (layer B.Cu) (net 12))
 (segment (start 128.905 31.75) (end 130.03637 31.75) (width 0.25) (layer B.Cu) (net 12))
 (segment (start 139.435 33.02) (end 140.705 31.75) (width 0.25) (layer B.Cu) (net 12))
 (segment (start 131.30637 33.02) (end 139.435 33.02) (width 0.25) (layer B.Cu) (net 12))
 (segment (start 127.49217 31.75) (end 128.905 31.75) (width 0.25) (layer B.Cu) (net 12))
 (segment (start 109.34 33.02) (end 126.22217 33.02) (width 0.25) (layer B.Cu) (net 12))
 (segment (start 126.22217 33.02) (end 127.49217 31.75) (width 0.25) (layer B.Cu) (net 12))
 (segment (start 128.905 39.37) (end 130.03637 39.37) (width 0.25) (layer B.Cu) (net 18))
 (segment (start 139.435 40.64) (end 140.705 39.37) (width 0.25) (layer B.Cu) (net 18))
 (segment (start 131.30637 40.64) (end 139.435 40.64) (width 0.25) (layer B.Cu) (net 18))
 (segment (start 130.03637 39.37) (end 131.30637 40.64) (width 0.25) (layer B.Cu) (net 18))
 (segment (start 116.84 40.64) (end 117.96717 40.64) (width 0.25) (layer B.Cu) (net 18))
 (segment (start 109.34 40.64) (end 116.84 40.64) (width 0.25) (layer B.Cu) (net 18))
 (segment (start 127.77363 39.37) (end 128.905 39.37) (width 0.25) (layer B.Cu) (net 18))
 (segment (start 116.84 40.64) (end 121.77717 40.64) (width 0.25) (layer B.Cu) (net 18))
 (segment (start 121.77717 40.64) (end 122.41217 40.005) (width 0.25) (layer B.Cu) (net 18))
 (segment (start 122.41217 40.005) (end 125.87283 40.005) (width 0.25) (layer B.Cu) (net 18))
 (segment (start 125.87283 40.005) (end 126.50783 39.37) (width 0.25) (layer B.Cu) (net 18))
 (segment (start 126.50783 39.37) (end 127.77363 39.37) (width 0.25) (layer B.Cu) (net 18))
 (segment (start 109.34 41.91) (end 109.855 41.91) (width 0.25) (layer B.Cu) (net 19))
 (segment (start 109.34 41.91) (end 121.285 41.91) (width 0.25) (layer B.Cu) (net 19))
 (segment (start 130.175 40.64) (end 131.445 41.91) (width 0.25) (layer B.Cu) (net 19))
 (segment (start 125.73 41.91) (end 127 40.64) (width 0.25) (layer B.Cu) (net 19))
 (segment (start 121.285 41.91) (end 125.73 41.91) (width 0.25) (layer B.Cu) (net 19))
 (segment (start 127 40.64) (end 128.27 40.64) (width 0.25) (layer B.Cu) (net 19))
 (segment (start 128.27 40.64) (end 128.905 40.64) (width 0.25) (layer B.Cu) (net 19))
 (segment (start 128.905 40.64) (end 130.175 40.64) (width 0.25) (layer B.Cu) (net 19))
 (segment (start 131.445 41.91) (end 133.085 41.91) (width 0.25) (layer B.Cu) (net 19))
 (segment (start 128.905 41.91) (end 130.175 41.91) (width 0.25) (layer B.Cu) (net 7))
 (segment (start 130.175 41.91) (end 131.445 43.18) (width 0.25) (layer B.Cu) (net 7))
 (segment (start 139.435 43.18) (end 140.705 41.91) (width 0.25) (layer B.Cu) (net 7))
 (segment (start 131.445 43.18) (end 139.435 43.18) (width 0.25) (layer B.Cu) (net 7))
 (segment (start 103.505 31.60717) (end 103.589992 31.522178) (width 0.25) (layer B.Cu) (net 7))
 (segment (start 103.589992 31.522178) (end 106.53717 28.575) (width 0.25) (layer B.Cu) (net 7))
 (segment (start 106.53717 28.575) (end 111.76 28.575) (width 0.25) (layer B.Cu) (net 7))
 (segment (start 111.76 28.575) (end 113.03 27.305) (width 0.25) (layer B.Cu) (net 7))
 (segment (start 113.03 27.305) (end 118.745 27.305) (width 0.25) (layer B.Cu) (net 7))
 (segment (start 144.145 38.47) (end 140.705 41.91) (width 0.25) (layer B.Cu) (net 7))
 (segment (start 143.01783 28.575) (end 144.145 29.70217) (width 0.25) (layer B.Cu) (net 7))
 (segment (start 118.745 27.305) (end 120.015 28.575) (width 0.25) (layer B.Cu) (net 7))
 (segment (start 144.145 29.70217) (end 144.145 38.47) (width 0.25) (layer B.Cu) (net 7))
 (segment (start 120.015 28.575) (end 143.01783 28.575) (width 0.25) (layer B.Cu) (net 7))
 (segment (start 98.94 35.56) (end 102.235 35.56) (width 0.25) (layer B.Cu) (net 7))
 (segment (start 102.235 35.56) (end 103.505 34.29) (width 0.25) (layer B.Cu) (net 7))
 (segment (start 103.505 34.29) (end 103.505 33.655) (width 0.25) (layer B.Cu) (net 7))
 (segment (start 103.505 33.655) (end 103.505 31.60717) (width 0.25) (layer B.Cu) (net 7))
 (segment (start 84.835 30.48) (end 83.185 28.83) (width 0.25) (layer B.Cu) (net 26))
 (segment (start 86.335 30.48) (end 84.835 30.48) (width 0.25) (layer B.Cu) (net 26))
 (segment (start 83.185 28.83) (end 83.185 26.17783) (width 0.25) (layer B.Cu) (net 26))
 (segment (start 83.185 26.17783) (end 83.04217 26.035) (width 0.25) (layer B.Cu) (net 26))
 (segment (start 83.04217 26.035) (end 73.66 26.035) (width 0.25) (layer B.Cu) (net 26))
 (segment (start 42.805239 30.667001) (end 69.027999 30.667001) (width 0.25) (layer B.Cu) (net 26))
 (segment (start 42.187999 30.049761) (end 42.805239 30.667001) (width 0.25) (layer B.Cu) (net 26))
 (segment (start 43.375 31.48) (end 42.187999 30.292999) (width 0.25) (layer B.Cu) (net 26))
 (segment (start 42.187999 30.292999) (end 42.187999 30.049761) (width 0.25) (layer B.Cu) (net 26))
 (segment (start 69.027999 30.667001) (end 73.66 26.035) (width 0.25) (layer B.Cu) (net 26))
 (segment (start 83.82 28.195) (end 84.835 29.21) (width 0.25) (layer B.Cu) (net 27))
 (segment (start 72.39 25.4) (end 83.185 25.4) (width 0.25) (layer B.Cu) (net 27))
 (segment (start 68.31 29.48) (end 72.39 25.4) (width 0.25) (layer B.Cu) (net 27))
 (segment (start 84.835 29.21) (end 86.335 29.21) (width 0.25) (layer B.Cu) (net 27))
 (segment (start 43.375 29.48) (end 68.31 29.48) (width 0.25) (layer B.Cu) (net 27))
 (segment (start 83.185 25.4) (end 83.82 26.035) (width 0.25) (layer B.Cu) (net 27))
 (segment (start 83.82 26.035) (end 83.82 28.195) (width 0.25) (layer B.Cu) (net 27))
 (segment (start 107.615 38.1) (end 109.34 38.1) (width 0.25) (layer B.Cu) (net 16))
 (segment (start 106.68 38.1) (end 107.615 38.1) (width 0.25) (layer B.Cu) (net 16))
 (segment (start 104.14 40.64) (end 106.68 38.1) (width 0.25) (layer B.Cu) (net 16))
 (segment (start 104.14 50.8) (end 104.14 40.64) (width 0.25) (layer B.Cu) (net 16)))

